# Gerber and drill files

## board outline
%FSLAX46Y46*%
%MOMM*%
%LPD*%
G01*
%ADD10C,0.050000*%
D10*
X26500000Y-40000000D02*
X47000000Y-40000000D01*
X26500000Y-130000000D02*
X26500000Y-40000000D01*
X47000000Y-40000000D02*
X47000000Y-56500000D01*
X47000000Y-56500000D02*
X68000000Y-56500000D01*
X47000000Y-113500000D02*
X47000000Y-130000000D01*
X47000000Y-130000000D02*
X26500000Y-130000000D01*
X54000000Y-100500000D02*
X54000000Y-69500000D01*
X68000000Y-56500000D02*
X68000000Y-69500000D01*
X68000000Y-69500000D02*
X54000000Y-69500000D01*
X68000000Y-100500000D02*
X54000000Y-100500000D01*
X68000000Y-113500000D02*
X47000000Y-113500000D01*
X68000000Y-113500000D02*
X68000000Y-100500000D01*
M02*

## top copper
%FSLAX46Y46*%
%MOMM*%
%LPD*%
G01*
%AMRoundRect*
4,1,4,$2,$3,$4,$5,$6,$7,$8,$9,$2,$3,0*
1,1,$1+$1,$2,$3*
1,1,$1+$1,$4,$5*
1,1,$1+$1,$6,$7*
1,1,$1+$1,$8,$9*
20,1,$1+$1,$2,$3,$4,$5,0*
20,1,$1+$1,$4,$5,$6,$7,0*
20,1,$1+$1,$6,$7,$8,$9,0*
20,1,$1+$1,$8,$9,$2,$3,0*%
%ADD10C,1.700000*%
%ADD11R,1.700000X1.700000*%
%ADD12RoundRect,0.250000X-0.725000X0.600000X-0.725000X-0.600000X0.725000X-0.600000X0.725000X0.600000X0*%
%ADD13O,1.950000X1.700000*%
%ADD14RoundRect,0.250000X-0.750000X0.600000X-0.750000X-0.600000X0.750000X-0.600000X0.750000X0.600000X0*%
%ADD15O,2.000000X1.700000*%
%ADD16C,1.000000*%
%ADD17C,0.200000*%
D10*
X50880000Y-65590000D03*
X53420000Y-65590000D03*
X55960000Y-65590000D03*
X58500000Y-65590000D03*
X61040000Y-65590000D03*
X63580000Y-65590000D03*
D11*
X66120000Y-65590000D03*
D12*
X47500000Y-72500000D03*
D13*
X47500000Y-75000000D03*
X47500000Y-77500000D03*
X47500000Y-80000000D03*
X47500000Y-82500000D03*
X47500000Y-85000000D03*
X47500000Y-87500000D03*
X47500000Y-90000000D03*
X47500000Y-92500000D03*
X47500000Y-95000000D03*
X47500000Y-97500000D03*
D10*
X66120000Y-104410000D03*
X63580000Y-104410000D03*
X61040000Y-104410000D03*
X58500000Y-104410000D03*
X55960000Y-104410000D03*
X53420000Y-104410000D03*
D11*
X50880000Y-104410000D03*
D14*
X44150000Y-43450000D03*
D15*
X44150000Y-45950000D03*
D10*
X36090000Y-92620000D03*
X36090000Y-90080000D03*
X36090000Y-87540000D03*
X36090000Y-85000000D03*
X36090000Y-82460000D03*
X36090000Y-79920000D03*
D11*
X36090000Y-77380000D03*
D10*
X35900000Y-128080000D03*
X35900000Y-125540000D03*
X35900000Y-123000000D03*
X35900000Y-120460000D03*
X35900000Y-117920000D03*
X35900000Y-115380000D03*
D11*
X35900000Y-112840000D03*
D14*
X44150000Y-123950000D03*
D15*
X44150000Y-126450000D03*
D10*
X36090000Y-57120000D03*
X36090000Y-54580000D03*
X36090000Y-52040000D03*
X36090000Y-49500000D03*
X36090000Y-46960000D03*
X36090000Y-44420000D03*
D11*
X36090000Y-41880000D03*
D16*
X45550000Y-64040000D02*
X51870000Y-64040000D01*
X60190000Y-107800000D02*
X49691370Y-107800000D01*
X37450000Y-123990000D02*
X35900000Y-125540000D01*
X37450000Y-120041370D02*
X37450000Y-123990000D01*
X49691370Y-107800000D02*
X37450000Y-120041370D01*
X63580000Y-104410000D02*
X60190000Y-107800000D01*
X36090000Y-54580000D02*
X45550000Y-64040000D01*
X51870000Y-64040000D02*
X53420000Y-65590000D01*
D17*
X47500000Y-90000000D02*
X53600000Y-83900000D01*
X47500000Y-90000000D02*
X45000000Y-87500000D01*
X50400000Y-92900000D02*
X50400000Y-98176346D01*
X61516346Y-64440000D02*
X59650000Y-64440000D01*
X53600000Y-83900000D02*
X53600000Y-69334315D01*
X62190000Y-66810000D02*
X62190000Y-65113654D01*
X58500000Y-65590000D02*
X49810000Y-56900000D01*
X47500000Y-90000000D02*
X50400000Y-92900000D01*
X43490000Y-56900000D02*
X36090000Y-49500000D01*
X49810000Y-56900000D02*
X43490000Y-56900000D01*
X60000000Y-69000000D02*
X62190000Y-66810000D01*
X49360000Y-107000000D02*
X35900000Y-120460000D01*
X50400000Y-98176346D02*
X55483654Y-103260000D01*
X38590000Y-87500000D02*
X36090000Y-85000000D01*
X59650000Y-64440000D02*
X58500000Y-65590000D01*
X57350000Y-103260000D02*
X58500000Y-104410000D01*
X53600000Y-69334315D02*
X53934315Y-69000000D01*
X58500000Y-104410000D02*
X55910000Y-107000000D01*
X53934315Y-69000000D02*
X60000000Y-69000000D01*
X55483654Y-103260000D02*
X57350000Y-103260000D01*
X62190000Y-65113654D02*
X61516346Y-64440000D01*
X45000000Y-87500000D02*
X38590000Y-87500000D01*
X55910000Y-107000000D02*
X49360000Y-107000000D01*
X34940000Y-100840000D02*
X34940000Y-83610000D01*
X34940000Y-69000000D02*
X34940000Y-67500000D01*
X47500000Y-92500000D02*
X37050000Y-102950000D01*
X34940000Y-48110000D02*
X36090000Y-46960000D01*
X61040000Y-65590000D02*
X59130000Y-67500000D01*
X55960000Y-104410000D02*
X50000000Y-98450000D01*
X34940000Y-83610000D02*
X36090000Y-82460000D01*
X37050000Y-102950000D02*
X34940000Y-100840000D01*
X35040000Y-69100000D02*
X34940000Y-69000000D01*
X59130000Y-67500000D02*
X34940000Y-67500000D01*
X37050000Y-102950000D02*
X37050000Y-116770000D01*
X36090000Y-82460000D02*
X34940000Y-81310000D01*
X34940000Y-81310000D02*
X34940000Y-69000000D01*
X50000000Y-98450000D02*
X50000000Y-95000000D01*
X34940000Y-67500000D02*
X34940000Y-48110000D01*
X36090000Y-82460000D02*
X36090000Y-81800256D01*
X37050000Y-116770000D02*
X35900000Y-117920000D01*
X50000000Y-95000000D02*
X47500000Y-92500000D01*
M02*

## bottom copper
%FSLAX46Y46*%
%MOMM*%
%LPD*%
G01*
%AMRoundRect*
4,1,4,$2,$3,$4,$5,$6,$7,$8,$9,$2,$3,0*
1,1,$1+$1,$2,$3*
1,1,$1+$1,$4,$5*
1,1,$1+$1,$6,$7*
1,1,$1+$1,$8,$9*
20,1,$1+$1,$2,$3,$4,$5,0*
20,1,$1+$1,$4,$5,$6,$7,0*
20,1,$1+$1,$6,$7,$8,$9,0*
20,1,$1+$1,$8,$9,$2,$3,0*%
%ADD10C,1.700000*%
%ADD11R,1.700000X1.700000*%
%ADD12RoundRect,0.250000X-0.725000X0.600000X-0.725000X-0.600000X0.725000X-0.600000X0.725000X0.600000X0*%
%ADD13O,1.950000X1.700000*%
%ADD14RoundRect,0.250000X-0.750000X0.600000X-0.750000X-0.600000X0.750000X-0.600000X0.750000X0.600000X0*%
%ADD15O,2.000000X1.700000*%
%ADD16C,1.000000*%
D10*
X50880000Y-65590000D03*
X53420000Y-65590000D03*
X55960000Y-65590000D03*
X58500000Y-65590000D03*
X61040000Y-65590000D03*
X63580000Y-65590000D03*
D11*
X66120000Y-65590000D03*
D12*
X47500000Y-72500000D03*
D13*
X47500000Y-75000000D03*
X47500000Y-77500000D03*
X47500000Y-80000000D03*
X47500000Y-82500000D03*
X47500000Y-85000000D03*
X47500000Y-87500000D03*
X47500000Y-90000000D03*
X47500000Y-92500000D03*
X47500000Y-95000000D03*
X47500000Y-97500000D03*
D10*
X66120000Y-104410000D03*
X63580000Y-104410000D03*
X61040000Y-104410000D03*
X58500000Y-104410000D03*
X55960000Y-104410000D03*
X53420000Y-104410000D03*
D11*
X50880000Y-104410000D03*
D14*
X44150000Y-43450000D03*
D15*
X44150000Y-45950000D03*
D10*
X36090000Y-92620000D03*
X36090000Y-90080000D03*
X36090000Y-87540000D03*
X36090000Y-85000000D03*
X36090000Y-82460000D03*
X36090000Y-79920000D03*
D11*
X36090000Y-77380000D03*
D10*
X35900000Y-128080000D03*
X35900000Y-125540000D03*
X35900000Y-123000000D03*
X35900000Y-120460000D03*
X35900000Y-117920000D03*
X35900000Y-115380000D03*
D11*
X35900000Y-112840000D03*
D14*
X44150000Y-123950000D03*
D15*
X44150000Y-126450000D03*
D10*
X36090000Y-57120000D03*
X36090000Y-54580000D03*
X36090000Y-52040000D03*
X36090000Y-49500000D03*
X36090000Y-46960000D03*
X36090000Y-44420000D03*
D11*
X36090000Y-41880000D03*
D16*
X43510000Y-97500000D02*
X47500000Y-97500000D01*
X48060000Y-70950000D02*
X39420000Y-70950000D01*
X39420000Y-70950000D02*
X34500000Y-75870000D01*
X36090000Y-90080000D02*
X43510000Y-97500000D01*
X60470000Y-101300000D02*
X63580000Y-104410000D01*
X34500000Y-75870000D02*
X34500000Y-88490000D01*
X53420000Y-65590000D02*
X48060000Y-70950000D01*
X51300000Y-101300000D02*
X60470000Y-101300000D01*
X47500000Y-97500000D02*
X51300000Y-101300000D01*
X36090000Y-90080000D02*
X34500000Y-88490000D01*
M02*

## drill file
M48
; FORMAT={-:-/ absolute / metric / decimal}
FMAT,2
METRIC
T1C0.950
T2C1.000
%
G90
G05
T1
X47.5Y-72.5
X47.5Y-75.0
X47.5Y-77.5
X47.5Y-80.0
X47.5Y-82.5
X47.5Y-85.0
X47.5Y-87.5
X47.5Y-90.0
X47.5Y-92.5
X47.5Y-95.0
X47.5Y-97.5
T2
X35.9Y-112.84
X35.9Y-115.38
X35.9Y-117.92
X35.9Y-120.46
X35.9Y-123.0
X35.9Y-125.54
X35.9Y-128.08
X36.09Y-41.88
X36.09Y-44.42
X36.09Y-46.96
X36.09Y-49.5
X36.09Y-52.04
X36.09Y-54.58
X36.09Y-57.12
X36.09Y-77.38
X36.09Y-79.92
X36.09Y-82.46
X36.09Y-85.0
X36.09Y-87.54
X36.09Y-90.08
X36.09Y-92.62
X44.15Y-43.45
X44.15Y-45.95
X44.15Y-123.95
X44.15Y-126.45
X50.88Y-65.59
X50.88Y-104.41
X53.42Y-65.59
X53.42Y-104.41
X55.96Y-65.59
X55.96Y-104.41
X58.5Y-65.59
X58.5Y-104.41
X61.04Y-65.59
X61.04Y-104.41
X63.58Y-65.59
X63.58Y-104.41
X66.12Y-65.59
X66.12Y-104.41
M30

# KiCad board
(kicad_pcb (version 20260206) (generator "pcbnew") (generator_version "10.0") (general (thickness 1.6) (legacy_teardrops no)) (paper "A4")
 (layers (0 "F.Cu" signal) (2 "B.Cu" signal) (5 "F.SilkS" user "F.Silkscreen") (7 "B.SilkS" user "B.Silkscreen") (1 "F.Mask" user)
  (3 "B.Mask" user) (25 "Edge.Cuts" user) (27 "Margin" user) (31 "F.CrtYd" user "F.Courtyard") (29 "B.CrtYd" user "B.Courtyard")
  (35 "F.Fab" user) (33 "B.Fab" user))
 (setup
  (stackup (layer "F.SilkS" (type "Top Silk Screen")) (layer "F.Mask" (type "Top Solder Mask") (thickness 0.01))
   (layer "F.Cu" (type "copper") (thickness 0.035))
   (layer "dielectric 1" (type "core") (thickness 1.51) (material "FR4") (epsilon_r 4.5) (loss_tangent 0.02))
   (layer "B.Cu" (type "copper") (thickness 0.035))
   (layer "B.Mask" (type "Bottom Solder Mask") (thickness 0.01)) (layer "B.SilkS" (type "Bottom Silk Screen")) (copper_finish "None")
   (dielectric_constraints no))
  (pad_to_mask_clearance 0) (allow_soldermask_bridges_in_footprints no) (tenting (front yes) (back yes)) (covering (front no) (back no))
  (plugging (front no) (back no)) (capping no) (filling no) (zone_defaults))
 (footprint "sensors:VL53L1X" (layer "F.Cu") (at 58.5 55.5 -90)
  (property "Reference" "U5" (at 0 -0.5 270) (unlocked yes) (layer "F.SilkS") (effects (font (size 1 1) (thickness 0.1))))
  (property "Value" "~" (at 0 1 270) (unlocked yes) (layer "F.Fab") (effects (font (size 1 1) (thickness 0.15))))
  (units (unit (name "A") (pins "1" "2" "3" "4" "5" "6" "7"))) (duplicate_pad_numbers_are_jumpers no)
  (pad "1" thru_hole circle (at 10.09 7.62 270) (size 1.7 1.7) (drill 1) (layers "*.Cu" "*.Mask") (remove_unused_layers no)
   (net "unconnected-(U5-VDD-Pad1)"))
  (pad "2" thru_hole circle (at 10.09 5.08 270) (size 1.7 1.7) (drill 1) (layers "*.Cu" "*.Mask") (remove_unused_layers no) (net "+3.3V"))
  (pad "3" thru_hole circle (at 10.09 2.54 270) (size 1.7 1.7) (drill 1) (layers "*.Cu" "*.Mask") (remove_unused_layers no)
   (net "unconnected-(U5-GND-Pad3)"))
  (pad "4" thru_hole circle (at 10.09 0 270) (size 1.7 1.7) (drill 1) (layers "*.Cu" "*.Mask") (remove_unused_layers no) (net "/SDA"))
  (pad "5" thru_hole circle (at 10.09 -2.54 270) (size 1.7 1.7) (drill 1) (layers "*.Cu" "*.Mask") (remove_unused_layers no) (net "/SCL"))
  (pad "6" thru_hole circle (at 10.09 -5.08 270) (size 1.7 1.7) (drill 1) (layers "*.Cu" "*.Mask") (remove_unused_layers no)
   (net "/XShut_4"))
  (pad "7" thru_hole rect (at 10.09 -7.62 270) (size 1.7 1.7) (drill 1) (layers "*.Cu" "*.Mask") (remove_unused_layers no)
   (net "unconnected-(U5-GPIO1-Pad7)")))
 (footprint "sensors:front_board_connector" (layer "F.Cu") (at 47.5 84.75 -90)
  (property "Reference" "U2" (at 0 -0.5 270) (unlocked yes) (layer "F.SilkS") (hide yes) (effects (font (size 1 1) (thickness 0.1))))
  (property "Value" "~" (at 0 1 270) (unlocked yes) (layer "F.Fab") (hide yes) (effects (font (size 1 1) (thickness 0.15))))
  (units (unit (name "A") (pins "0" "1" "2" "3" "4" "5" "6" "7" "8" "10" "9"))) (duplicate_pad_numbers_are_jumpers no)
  (pad "0" thru_hole roundrect (at -12.25 0 270) (size 1.7 1.95) (drill 0.95) (layers "*.Cu" "*.Mask") (remove_unused_layers no)
   (roundrect_rratio 0.147059) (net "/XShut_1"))
  (pad "1" thru_hole oval (at -9.75 0 270) (size 1.7 1.95) (drill 0.95) (layers "*.Cu" "*.Mask") (remove_unused_layers no) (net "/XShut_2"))
  (pad "2" thru_hole oval (at -7.25 0 270) (size 1.7 1.95) (drill 0.95) (layers "*.Cu" "*.Mask") (remove_unused_layers no) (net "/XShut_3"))
  (pad "3" thru_hole oval (at -4.75 0 270) (size 1.7 1.95) (drill 0.95) (layers "*.Cu" "*.Mask") (remove_unused_layers no) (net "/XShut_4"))
  (pad "4" thru_hole oval (at -2.25 0 270) (size 1.7 1.95) (drill 0.95) (layers "*.Cu" "*.Mask") (remove_unused_layers no) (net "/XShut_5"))
  (pad "5" thru_hole oval (at 0.25 0 270) (size 1.7 1.95) (drill 0.95) (layers "*.Cu" "*.Mask") (remove_unused_layers no)
   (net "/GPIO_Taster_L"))
  (pad "6" thru_hole oval (at 2.75 0 270) (size 1.7 1.95) (drill 0.95) (layers "*.Cu" "*.Mask") (remove_unused_layers no)
   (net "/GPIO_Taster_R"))
  (pad "7" thru_hole oval (at 5.25 0 270) (size 1.7 1.95) (drill 0.95) (layers "*.Cu" "*.Mask") (remove_unused_layers no) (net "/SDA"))
  (pad "8" thru_hole oval (at 7.75 0 270) (size 1.7 1.95) (drill 0.95) (layers "*.Cu" "*.Mask") (remove_unused_layers no) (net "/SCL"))
  (pad "9" thru_hole oval (at 10.25 0 270) (size 1.7 1.95) (drill 0.95) (layers "*.Cu" "*.Mask") (remove_unused_layers no) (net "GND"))
  (pad "10" thru_hole oval (at 12.75 0 270) (size 1.7 1.95) (drill 0.95) (layers "*.Cu" "*.Mask") (remove_unused_layers no) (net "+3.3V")))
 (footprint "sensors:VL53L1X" (layer "F.Cu") (at 58.5 114.5 90)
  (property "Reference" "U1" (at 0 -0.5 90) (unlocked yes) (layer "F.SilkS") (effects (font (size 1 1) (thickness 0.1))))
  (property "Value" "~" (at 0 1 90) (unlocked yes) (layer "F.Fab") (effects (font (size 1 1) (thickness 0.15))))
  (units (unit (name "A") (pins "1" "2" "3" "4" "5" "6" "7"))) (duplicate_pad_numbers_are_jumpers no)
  (pad "1" thru_hole circle (at 10.09 7.62 90) (size 1.7 1.7) (drill 1) (layers "*.Cu" "*.Mask") (remove_unused_layers no)
   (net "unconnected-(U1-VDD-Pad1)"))
  (pad "2" thru_hole circle (at 10.09 5.08 90) (size 1.7 1.7) (drill 1) (layers "*.Cu" "*.Mask") (remove_unused_layers no) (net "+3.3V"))
  (pad "3" thru_hole circle (at 10.09 2.54 90) (size 1.7 1.7) (drill 1) (layers "*.Cu" "*.Mask") (remove_unused_layers no) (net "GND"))
  (pad "4" thru_hole circle (at 10.09 0 90) (size 1.7 1.7) (drill 1) (layers "*.Cu" "*.Mask") (remove_unused_layers no) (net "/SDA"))
  (pad "5" thru_hole circle (at 10.09 -2.54 90) (size 1.7 1.7) (drill 1) (layers "*.Cu" "*.Mask") (remove_unused_layers no) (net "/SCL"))
  (pad "6" thru_hole circle (at 10.09 -5.08 90) (size 1.7 1.7) (drill 1) (layers "*.Cu" "*.Mask") (remove_unused_layers no) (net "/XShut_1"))
  (pad "7" thru_hole rect (at 10.09 -7.62 90) (size 1.7 1.7) (drill 1) (layers "*.Cu" "*.Mask") (remove_unused_layers no)
   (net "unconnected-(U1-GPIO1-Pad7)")))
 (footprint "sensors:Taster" (layer "F.Cu") (at 43.5 44.5 -90)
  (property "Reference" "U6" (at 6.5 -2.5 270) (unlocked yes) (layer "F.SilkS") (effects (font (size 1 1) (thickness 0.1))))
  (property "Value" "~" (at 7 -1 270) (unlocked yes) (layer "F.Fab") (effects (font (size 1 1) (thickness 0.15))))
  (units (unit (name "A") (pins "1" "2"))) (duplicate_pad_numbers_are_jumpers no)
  (pad "1" thru_hole roundrect (at -1.05 -0.65 270) (size 1.7 2) (drill 1) (layers "*.Cu" "*.Mask") (remove_unused_layers no)
   (roundrect_rratio 0.147059) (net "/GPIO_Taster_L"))
  (pad "2" thru_hole oval (at 1.45 -0.65 270) (size 1.7 2) (drill 1) (layers "*.Cu" "*.Mask") (remove_unused_layers no) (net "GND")))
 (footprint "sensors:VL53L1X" (layer "F.Cu") (at 26 85)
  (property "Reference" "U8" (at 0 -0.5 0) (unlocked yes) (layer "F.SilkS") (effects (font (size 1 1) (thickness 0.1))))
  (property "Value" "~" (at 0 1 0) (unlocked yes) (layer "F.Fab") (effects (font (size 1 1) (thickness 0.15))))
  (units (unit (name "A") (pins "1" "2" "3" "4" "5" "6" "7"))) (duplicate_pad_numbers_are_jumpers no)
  (pad "1" thru_hole circle (at 10.09 7.62) (size 1.7 1.7) (drill 1) (layers "*.Cu" "*.Mask") (remove_unused_layers no)
   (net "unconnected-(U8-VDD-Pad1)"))
  (pad "2" thru_hole circle (at 10.09 5.08) (size 1.7 1.7) (drill 1) (layers "*.Cu" "*.Mask") (remove_unused_layers no) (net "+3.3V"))
  (pad "3" thru_hole circle (at 10.09 2.54) (size 1.7 1.7) (drill 1) (layers "*.Cu" "*.Mask") (remove_unused_layers no) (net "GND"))
  (pad "4" thru_hole circle (at 10.09 0) (size 1.7 1.7) (drill 1) (layers "*.Cu" "*.Mask") (remove_unused_layers no) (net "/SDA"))
  (pad "5" thru_hole circle (at 10.09 -2.54) (size 1.7 1.7) (drill 1) (layers "*.Cu" "*.Mask") (remove_unused_layers no) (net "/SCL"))
  (pad "6" thru_hole circle (at 10.09 -5.08) (size 1.7 1.7) (drill 1) (layers "*.Cu" "*.Mask") (remove_unused_layers no) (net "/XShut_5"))
  (pad "7" thru_hole rect (at 10.09 -7.62) (size 1.7 1.7) (drill 1) (layers "*.Cu" "*.Mask") (remove_unused_layers no)
   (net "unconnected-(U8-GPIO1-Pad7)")))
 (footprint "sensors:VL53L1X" (layer "F.Cu") (at 25.81 120.46)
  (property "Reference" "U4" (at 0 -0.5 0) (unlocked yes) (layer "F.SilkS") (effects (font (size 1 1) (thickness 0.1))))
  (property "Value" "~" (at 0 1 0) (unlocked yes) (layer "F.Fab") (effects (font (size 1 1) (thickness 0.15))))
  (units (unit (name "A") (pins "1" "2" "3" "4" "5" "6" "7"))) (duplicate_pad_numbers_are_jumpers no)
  (pad "1" thru_hole circle (at 10.09 7.62) (size 1.7 1.7) (drill 1) (layers "*.Cu" "*.Mask") (remove_unused_layers no)
   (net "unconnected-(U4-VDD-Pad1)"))
  (pad "2" thru_hole circle (at 10.09 5.08) (size 1.7 1.7) (drill 1) (layers "*.Cu" "*.Mask") (remove_unused_layers no) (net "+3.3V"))
  (pad "3" thru_hole circle (at 10.09 2.54) (size 1.7 1.7) (drill 1) (layers "*.Cu" "*.Mask") (remove_unused_layers no) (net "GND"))
  (pad "4" thru_hole circle (at 10.09 0) (size 1.7 1.7) (drill 1) (layers "*.Cu" "*.Mask") (remove_unused_layers no) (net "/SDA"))
  (pad "5" thru_hole circle (at 10.09 -2.54) (size 1.7 1.7) (drill 1) (layers "*.Cu" "*.Mask") (remove_unused_layers no) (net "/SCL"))
  (pad "6" thru_hole circle (at 10.09 -5.08) (size 1.7 1.7) (drill 1) (layers "*.Cu" "*.Mask") (remove_unused_layers no) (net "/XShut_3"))
  (pad "7" thru_hole rect (at 10.09 -7.62) (size 1.7 1.7) (drill 1) (layers "*.Cu" "*.Mask") (remove_unused_layers no)
   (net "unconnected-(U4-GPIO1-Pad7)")))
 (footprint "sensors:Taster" (layer "F.Cu") (at 43.5 125 -90)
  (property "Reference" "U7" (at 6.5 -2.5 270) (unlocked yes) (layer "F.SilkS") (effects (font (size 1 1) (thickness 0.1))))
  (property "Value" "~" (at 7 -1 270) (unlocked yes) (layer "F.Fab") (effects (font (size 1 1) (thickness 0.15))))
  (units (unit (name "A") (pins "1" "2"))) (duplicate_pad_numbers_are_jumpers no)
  (pad "1" thru_hole roundrect (at -1.05 -0.65 270) (size 1.7 2) (drill 1) (layers "*.Cu" "*.Mask") (remove_unused_layers no)
   (roundrect_rratio 0.147059) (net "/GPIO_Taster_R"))
  (pad "2" thru_hole oval (at 1.45 -0.65 270) (size 1.7 2) (drill 1) (layers "*.Cu" "*.Mask") (remove_unused_layers no) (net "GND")))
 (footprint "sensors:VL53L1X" (layer "F.Cu") (at 26 49.5)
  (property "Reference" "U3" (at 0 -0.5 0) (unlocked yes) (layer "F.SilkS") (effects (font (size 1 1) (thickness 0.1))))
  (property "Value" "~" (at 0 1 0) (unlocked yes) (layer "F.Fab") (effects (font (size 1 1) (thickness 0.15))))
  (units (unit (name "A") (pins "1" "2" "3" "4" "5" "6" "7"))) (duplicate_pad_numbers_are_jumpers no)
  (pad "1" thru_hole circle (at 10.09 7.62) (size 1.7 1.7) (drill 1) (layers "*.Cu" "*.Mask") (remove_unused_layers no)
   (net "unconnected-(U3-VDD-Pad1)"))
  (pad "2" thru_hole circle (at 10.09 5.08) (size 1.7 1.7) (drill 1) (layers "*.Cu" "*.Mask") (remove_unused_layers no) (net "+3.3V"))
  (pad "3" thru_hole circle (at 10.09 2.54) (size 1.7 1.7) (drill 1) (layers "*.Cu" "*.Mask") (remove_unused_layers no) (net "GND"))
  (pad "4" thru_hole circle (at 10.09 0) (size 1.7 1.7) (drill 1) (layers "*.Cu" "*.Mask") (remove_unused_layers no) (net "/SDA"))
  (pad "5" thru_hole circle (at 10.09 -2.54) (size 1.7 1.7) (drill 1) (layers "*.Cu" "*.Mask") (remove_unused_layers no) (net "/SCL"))
  (pad "6" thru_hole circle (at 10.09 -5.08) (size 1.7 1.7) (drill 1) (layers "*.Cu" "*.Mask") (remove_unused_layers no) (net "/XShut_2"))
  (pad "7" thru_hole rect (at 10.09 -7.62) (size 1.7 1.7) (drill 1) (layers "*.Cu" "*.Mask") (remove_unused_layers no)
   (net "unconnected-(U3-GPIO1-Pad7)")))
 (gr_line (start 26.5 40) (end 47 40) (stroke (width 0.05) (type default)) (layer "Edge.Cuts"))
 (gr_line (start 26.5 130) (end 26.5 40) (stroke (width 0.05) (type default)) (layer "Edge.Cuts"))
 (gr_line (start 47 40) (end 47 56.5) (stroke (width 0.05) (type default)) (layer "Edge.Cuts"))
 (gr_line (start 47 56.5) (end 68 56.5) (stroke (width 0.05) (type default)) (layer "Edge.Cuts"))
 (gr_line (start 47 113.5) (end 47 130) (stroke (width 0.05) (type default)) (layer "Edge.Cuts"))
 (gr_line (start 47 130) (end 26.5 130) (stroke (width 0.05) (type default)) (layer "Edge.Cuts"))
 (gr_line (start 54 100.5) (end 54 69.5) (stroke (width 0.05) (type default)) (layer "Edge.Cuts"))
 (gr_line (start 68 56.5) (end 68 69.5) (stroke (width 0.05) (type default)) (layer "Edge.Cuts"))
 (gr_line (start 68 69.5) (end 54 69.5) (stroke (width 0.05) (type default)) (layer "Edge.Cuts"))
 (gr_line (start 68 100.5) (end 54 100.5) (stroke (width 0.05) (type default)) (layer "Edge.Cuts"))
 (gr_line (start 68 113.5) (end 47 113.5) (stroke (width 0.05) (type default)) (layer "Edge.Cuts"))
 (gr_line (start 68 113.5) (end 68 100.5) (stroke (width 0.05) (type default)) (layer "Edge.Cuts"))
 (segment (start 45.55 64.04) (end 51.87 64.04) (width 1) (layer "F.Cu") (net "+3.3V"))
 (segment (start 60.19 107.8) (end 49.69137 107.8) (width 1) (layer "F.Cu") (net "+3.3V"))
 (segment (start 37.45 123.99) (end 35.9 125.54) (width 1) (layer "F.Cu") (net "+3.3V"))
 (segment (start 37.45 120.04137) (end 37.45 123.99) (width 1) (layer "F.Cu") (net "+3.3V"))
 (segment (start 49.69137 107.8) (end 37.45 120.04137) (width 1) (layer "F.Cu") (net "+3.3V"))
 (segment (start 63.58 104.41) (end 60.19 107.8) (width 1) (layer "F.Cu") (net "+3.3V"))
 (segment (start 36.09 54.58) (end 45.55 64.04) (width 1) (layer "F.Cu") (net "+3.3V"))
 (segment (start 51.87 64.04) (end 53.42 65.59) (width 1) (layer "F.Cu") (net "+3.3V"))
 (segment (start 43.51 97.5) (end 47.5 97.5) (width 1) (layer "B.Cu") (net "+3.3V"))
 (segment (start 48.06 70.95) (end 39.42 70.95) (width 1) (layer "B.Cu") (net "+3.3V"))
 (segment (start 39.42 70.95) (end 34.5 75.87) (width 1) (layer "B.Cu") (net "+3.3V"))
 (segment (start 36.09 90.08) (end 43.51 97.5) (width 1) (layer "B.Cu") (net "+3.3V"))
 (segment (start 60.47 101.3) (end 63.58 104.41) (width 1) (layer "B.Cu") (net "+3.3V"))
 (segment (start 34.5 75.87) (end 34.5 88.49) (width 1) (layer "B.Cu") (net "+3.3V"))
 (segment (start 53.42 65.59) (end 48.06 70.95) (width 1) (layer "B.Cu") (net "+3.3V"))
 (segment (start 51.3 101.3) (end 60.47 101.3) (width 1) (layer "B.Cu") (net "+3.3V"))
 (segment (start 47.5 97.5) (end 51.3 101.3) (width 1) (layer "B.Cu") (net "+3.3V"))
 (segment (start 36.09 90.08) (end 34.5 88.49) (width 1) (layer "B.Cu") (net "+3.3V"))
 (segment (start 47.5 90) (end 53.6 83.9) (width 0.2) (layer "F.Cu") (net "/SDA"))
 (segment (start 47.5 90) (end 45 87.5) (width 0.2) (layer "F.Cu") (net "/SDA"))
 (segment (start 50.4 92.9) (end 50.4 98.176346) (width 0.2) (layer "F.Cu") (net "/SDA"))
 (segment (start 61.516346 64.44) (end 59.65 64.44) (width 0.2) (layer "F.Cu") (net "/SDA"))
 (segment (start 53.6 83.9) (end 53.6 69.334315) (width 0.2) (layer "F.Cu") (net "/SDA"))
 (segment (start 62.19 66.81) (end 62.19 65.113654) (width 0.2) (layer "F.Cu") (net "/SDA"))
 (segment (start 58.5 65.59) (end 49.81 56.9) (width 0.2) (layer "F.Cu") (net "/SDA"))
 (segment (start 47.5 90) (end 50.4 92.9) (width 0.2) (layer "F.Cu") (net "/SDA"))
 (segment (start 43.49 56.9) (end 36.09 49.5) (width 0.2) (layer "F.Cu") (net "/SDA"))
 (segment (start 49.81 56.9) (end 43.49 56.9) (width 0.2) (layer "F.Cu") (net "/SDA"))
 (segment (start 60 69) (end 62.19 66.81) (width 0.2) (layer "F.Cu") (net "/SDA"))
 (segment (start 49.36 107) (end 35.9 120.46) (width 0.2) (layer "F.Cu") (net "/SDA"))
 (segment (start 50.4 98.176346) (end 55.483654 103.26) (width 0.2) (layer "F.Cu") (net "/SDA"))
 (segment (start 38.59 87.5) (end 36.09 85) (width 0.2) (layer "F.Cu") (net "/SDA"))
 (segment (start 59.65 64.44) (end 58.5 65.59) (width 0.2) (layer "F.Cu") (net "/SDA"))
 (segment (start 57.35 103.26) (end 58.5 104.41) (width 0.2) (layer "F.Cu") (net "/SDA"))
 (segment (start 53.6 69.334315) (end 53.934315 69) (width 0.2) (layer "F.Cu") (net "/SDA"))
 (segment (start 58.5 104.41) (end 55.91 107) (width 0.2) (layer "F.Cu") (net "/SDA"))
 (segment (start 53.934315 69) (end 60 69) (width 0.2) (layer "F.Cu") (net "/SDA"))
 (segment (start 55.483654 103.26) (end 57.35 103.26) (width 0.2) (layer "F.Cu") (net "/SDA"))
 (segment (start 62.19 65.113654) (end 61.516346 64.44) (width 0.2) (layer "F.Cu") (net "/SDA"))
 (segment (start 45 87.5) (end 38.59 87.5) (width 0.2) (layer "F.Cu") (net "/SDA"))
 (segment (start 55.91 107) (end 49.36 107) (width 0.2) (layer "F.Cu") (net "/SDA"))
 (segment (start 34.94 100.84) (end 34.94 83.61) (width 0.2) (layer "F.Cu") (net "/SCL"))
 (segment (start 34.94 69) (end 34.94 67.5) (width 0.2) (layer "F.Cu") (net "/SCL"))
 (segment (start 47.5 92.5) (end 37.05 102.95) (width 0.2) (layer "F.Cu") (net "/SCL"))
 (segment (start 34.94 48.11) (end 36.09 46.96) (width 0.2) (layer "F.Cu") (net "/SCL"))
 (segment (start 61.04 65.59) (end 59.13 67.5) (width 0.2) (layer "F.Cu") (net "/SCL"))
 (segment (start 55.96 104.41) (end 50 98.45) (width 0.2) (layer "F.Cu") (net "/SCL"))
 (segment (start 34.94 83.61) (end 36.09 82.46) (width 0.2) (layer "F.Cu") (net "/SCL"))
 (segment (start 37.05 102.95) (end 34.94 100.84) (width 0.2) (layer "F.Cu") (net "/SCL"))
 (segment (start 35.04 69.1) (end 34.94 69) (width 0.2) (layer "F.Cu") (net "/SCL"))
 (segment (start 59.13 67.5) (end 34.94 67.5) (width 0.2) (layer "F.Cu") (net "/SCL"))
 (segment (start 37.05 102.95) (end 37.05 116.77) (width 0.2) (layer "F.Cu") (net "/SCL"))
 (segment (start 36.09 82.46) (end 34.94 81.31) (width 0.2) (layer "F.Cu") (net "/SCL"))
 (segment (start 34.94 81.31) (end 34.94 69) (width 0.2) (layer "F.Cu") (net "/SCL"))
 (segment (start 50 98.45) (end 50 95) (width 0.2) (layer "F.Cu") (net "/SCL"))
 (segment (start 34.94 67.5) (end 34.94 48.11) (width 0.2) (layer "F.Cu") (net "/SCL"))
 (segment (start 36.09 82.46) (end 36.09 81.800256) (width 0.2) (layer "F.Cu") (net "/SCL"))
 (segment (start 37.05 116.77) (end 35.9 117.92) (width 0.2) (layer "F.Cu") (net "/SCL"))
 (segment (start 50 95) (end 47.5 92.5) (width 0.2) (layer "F.Cu") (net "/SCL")))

